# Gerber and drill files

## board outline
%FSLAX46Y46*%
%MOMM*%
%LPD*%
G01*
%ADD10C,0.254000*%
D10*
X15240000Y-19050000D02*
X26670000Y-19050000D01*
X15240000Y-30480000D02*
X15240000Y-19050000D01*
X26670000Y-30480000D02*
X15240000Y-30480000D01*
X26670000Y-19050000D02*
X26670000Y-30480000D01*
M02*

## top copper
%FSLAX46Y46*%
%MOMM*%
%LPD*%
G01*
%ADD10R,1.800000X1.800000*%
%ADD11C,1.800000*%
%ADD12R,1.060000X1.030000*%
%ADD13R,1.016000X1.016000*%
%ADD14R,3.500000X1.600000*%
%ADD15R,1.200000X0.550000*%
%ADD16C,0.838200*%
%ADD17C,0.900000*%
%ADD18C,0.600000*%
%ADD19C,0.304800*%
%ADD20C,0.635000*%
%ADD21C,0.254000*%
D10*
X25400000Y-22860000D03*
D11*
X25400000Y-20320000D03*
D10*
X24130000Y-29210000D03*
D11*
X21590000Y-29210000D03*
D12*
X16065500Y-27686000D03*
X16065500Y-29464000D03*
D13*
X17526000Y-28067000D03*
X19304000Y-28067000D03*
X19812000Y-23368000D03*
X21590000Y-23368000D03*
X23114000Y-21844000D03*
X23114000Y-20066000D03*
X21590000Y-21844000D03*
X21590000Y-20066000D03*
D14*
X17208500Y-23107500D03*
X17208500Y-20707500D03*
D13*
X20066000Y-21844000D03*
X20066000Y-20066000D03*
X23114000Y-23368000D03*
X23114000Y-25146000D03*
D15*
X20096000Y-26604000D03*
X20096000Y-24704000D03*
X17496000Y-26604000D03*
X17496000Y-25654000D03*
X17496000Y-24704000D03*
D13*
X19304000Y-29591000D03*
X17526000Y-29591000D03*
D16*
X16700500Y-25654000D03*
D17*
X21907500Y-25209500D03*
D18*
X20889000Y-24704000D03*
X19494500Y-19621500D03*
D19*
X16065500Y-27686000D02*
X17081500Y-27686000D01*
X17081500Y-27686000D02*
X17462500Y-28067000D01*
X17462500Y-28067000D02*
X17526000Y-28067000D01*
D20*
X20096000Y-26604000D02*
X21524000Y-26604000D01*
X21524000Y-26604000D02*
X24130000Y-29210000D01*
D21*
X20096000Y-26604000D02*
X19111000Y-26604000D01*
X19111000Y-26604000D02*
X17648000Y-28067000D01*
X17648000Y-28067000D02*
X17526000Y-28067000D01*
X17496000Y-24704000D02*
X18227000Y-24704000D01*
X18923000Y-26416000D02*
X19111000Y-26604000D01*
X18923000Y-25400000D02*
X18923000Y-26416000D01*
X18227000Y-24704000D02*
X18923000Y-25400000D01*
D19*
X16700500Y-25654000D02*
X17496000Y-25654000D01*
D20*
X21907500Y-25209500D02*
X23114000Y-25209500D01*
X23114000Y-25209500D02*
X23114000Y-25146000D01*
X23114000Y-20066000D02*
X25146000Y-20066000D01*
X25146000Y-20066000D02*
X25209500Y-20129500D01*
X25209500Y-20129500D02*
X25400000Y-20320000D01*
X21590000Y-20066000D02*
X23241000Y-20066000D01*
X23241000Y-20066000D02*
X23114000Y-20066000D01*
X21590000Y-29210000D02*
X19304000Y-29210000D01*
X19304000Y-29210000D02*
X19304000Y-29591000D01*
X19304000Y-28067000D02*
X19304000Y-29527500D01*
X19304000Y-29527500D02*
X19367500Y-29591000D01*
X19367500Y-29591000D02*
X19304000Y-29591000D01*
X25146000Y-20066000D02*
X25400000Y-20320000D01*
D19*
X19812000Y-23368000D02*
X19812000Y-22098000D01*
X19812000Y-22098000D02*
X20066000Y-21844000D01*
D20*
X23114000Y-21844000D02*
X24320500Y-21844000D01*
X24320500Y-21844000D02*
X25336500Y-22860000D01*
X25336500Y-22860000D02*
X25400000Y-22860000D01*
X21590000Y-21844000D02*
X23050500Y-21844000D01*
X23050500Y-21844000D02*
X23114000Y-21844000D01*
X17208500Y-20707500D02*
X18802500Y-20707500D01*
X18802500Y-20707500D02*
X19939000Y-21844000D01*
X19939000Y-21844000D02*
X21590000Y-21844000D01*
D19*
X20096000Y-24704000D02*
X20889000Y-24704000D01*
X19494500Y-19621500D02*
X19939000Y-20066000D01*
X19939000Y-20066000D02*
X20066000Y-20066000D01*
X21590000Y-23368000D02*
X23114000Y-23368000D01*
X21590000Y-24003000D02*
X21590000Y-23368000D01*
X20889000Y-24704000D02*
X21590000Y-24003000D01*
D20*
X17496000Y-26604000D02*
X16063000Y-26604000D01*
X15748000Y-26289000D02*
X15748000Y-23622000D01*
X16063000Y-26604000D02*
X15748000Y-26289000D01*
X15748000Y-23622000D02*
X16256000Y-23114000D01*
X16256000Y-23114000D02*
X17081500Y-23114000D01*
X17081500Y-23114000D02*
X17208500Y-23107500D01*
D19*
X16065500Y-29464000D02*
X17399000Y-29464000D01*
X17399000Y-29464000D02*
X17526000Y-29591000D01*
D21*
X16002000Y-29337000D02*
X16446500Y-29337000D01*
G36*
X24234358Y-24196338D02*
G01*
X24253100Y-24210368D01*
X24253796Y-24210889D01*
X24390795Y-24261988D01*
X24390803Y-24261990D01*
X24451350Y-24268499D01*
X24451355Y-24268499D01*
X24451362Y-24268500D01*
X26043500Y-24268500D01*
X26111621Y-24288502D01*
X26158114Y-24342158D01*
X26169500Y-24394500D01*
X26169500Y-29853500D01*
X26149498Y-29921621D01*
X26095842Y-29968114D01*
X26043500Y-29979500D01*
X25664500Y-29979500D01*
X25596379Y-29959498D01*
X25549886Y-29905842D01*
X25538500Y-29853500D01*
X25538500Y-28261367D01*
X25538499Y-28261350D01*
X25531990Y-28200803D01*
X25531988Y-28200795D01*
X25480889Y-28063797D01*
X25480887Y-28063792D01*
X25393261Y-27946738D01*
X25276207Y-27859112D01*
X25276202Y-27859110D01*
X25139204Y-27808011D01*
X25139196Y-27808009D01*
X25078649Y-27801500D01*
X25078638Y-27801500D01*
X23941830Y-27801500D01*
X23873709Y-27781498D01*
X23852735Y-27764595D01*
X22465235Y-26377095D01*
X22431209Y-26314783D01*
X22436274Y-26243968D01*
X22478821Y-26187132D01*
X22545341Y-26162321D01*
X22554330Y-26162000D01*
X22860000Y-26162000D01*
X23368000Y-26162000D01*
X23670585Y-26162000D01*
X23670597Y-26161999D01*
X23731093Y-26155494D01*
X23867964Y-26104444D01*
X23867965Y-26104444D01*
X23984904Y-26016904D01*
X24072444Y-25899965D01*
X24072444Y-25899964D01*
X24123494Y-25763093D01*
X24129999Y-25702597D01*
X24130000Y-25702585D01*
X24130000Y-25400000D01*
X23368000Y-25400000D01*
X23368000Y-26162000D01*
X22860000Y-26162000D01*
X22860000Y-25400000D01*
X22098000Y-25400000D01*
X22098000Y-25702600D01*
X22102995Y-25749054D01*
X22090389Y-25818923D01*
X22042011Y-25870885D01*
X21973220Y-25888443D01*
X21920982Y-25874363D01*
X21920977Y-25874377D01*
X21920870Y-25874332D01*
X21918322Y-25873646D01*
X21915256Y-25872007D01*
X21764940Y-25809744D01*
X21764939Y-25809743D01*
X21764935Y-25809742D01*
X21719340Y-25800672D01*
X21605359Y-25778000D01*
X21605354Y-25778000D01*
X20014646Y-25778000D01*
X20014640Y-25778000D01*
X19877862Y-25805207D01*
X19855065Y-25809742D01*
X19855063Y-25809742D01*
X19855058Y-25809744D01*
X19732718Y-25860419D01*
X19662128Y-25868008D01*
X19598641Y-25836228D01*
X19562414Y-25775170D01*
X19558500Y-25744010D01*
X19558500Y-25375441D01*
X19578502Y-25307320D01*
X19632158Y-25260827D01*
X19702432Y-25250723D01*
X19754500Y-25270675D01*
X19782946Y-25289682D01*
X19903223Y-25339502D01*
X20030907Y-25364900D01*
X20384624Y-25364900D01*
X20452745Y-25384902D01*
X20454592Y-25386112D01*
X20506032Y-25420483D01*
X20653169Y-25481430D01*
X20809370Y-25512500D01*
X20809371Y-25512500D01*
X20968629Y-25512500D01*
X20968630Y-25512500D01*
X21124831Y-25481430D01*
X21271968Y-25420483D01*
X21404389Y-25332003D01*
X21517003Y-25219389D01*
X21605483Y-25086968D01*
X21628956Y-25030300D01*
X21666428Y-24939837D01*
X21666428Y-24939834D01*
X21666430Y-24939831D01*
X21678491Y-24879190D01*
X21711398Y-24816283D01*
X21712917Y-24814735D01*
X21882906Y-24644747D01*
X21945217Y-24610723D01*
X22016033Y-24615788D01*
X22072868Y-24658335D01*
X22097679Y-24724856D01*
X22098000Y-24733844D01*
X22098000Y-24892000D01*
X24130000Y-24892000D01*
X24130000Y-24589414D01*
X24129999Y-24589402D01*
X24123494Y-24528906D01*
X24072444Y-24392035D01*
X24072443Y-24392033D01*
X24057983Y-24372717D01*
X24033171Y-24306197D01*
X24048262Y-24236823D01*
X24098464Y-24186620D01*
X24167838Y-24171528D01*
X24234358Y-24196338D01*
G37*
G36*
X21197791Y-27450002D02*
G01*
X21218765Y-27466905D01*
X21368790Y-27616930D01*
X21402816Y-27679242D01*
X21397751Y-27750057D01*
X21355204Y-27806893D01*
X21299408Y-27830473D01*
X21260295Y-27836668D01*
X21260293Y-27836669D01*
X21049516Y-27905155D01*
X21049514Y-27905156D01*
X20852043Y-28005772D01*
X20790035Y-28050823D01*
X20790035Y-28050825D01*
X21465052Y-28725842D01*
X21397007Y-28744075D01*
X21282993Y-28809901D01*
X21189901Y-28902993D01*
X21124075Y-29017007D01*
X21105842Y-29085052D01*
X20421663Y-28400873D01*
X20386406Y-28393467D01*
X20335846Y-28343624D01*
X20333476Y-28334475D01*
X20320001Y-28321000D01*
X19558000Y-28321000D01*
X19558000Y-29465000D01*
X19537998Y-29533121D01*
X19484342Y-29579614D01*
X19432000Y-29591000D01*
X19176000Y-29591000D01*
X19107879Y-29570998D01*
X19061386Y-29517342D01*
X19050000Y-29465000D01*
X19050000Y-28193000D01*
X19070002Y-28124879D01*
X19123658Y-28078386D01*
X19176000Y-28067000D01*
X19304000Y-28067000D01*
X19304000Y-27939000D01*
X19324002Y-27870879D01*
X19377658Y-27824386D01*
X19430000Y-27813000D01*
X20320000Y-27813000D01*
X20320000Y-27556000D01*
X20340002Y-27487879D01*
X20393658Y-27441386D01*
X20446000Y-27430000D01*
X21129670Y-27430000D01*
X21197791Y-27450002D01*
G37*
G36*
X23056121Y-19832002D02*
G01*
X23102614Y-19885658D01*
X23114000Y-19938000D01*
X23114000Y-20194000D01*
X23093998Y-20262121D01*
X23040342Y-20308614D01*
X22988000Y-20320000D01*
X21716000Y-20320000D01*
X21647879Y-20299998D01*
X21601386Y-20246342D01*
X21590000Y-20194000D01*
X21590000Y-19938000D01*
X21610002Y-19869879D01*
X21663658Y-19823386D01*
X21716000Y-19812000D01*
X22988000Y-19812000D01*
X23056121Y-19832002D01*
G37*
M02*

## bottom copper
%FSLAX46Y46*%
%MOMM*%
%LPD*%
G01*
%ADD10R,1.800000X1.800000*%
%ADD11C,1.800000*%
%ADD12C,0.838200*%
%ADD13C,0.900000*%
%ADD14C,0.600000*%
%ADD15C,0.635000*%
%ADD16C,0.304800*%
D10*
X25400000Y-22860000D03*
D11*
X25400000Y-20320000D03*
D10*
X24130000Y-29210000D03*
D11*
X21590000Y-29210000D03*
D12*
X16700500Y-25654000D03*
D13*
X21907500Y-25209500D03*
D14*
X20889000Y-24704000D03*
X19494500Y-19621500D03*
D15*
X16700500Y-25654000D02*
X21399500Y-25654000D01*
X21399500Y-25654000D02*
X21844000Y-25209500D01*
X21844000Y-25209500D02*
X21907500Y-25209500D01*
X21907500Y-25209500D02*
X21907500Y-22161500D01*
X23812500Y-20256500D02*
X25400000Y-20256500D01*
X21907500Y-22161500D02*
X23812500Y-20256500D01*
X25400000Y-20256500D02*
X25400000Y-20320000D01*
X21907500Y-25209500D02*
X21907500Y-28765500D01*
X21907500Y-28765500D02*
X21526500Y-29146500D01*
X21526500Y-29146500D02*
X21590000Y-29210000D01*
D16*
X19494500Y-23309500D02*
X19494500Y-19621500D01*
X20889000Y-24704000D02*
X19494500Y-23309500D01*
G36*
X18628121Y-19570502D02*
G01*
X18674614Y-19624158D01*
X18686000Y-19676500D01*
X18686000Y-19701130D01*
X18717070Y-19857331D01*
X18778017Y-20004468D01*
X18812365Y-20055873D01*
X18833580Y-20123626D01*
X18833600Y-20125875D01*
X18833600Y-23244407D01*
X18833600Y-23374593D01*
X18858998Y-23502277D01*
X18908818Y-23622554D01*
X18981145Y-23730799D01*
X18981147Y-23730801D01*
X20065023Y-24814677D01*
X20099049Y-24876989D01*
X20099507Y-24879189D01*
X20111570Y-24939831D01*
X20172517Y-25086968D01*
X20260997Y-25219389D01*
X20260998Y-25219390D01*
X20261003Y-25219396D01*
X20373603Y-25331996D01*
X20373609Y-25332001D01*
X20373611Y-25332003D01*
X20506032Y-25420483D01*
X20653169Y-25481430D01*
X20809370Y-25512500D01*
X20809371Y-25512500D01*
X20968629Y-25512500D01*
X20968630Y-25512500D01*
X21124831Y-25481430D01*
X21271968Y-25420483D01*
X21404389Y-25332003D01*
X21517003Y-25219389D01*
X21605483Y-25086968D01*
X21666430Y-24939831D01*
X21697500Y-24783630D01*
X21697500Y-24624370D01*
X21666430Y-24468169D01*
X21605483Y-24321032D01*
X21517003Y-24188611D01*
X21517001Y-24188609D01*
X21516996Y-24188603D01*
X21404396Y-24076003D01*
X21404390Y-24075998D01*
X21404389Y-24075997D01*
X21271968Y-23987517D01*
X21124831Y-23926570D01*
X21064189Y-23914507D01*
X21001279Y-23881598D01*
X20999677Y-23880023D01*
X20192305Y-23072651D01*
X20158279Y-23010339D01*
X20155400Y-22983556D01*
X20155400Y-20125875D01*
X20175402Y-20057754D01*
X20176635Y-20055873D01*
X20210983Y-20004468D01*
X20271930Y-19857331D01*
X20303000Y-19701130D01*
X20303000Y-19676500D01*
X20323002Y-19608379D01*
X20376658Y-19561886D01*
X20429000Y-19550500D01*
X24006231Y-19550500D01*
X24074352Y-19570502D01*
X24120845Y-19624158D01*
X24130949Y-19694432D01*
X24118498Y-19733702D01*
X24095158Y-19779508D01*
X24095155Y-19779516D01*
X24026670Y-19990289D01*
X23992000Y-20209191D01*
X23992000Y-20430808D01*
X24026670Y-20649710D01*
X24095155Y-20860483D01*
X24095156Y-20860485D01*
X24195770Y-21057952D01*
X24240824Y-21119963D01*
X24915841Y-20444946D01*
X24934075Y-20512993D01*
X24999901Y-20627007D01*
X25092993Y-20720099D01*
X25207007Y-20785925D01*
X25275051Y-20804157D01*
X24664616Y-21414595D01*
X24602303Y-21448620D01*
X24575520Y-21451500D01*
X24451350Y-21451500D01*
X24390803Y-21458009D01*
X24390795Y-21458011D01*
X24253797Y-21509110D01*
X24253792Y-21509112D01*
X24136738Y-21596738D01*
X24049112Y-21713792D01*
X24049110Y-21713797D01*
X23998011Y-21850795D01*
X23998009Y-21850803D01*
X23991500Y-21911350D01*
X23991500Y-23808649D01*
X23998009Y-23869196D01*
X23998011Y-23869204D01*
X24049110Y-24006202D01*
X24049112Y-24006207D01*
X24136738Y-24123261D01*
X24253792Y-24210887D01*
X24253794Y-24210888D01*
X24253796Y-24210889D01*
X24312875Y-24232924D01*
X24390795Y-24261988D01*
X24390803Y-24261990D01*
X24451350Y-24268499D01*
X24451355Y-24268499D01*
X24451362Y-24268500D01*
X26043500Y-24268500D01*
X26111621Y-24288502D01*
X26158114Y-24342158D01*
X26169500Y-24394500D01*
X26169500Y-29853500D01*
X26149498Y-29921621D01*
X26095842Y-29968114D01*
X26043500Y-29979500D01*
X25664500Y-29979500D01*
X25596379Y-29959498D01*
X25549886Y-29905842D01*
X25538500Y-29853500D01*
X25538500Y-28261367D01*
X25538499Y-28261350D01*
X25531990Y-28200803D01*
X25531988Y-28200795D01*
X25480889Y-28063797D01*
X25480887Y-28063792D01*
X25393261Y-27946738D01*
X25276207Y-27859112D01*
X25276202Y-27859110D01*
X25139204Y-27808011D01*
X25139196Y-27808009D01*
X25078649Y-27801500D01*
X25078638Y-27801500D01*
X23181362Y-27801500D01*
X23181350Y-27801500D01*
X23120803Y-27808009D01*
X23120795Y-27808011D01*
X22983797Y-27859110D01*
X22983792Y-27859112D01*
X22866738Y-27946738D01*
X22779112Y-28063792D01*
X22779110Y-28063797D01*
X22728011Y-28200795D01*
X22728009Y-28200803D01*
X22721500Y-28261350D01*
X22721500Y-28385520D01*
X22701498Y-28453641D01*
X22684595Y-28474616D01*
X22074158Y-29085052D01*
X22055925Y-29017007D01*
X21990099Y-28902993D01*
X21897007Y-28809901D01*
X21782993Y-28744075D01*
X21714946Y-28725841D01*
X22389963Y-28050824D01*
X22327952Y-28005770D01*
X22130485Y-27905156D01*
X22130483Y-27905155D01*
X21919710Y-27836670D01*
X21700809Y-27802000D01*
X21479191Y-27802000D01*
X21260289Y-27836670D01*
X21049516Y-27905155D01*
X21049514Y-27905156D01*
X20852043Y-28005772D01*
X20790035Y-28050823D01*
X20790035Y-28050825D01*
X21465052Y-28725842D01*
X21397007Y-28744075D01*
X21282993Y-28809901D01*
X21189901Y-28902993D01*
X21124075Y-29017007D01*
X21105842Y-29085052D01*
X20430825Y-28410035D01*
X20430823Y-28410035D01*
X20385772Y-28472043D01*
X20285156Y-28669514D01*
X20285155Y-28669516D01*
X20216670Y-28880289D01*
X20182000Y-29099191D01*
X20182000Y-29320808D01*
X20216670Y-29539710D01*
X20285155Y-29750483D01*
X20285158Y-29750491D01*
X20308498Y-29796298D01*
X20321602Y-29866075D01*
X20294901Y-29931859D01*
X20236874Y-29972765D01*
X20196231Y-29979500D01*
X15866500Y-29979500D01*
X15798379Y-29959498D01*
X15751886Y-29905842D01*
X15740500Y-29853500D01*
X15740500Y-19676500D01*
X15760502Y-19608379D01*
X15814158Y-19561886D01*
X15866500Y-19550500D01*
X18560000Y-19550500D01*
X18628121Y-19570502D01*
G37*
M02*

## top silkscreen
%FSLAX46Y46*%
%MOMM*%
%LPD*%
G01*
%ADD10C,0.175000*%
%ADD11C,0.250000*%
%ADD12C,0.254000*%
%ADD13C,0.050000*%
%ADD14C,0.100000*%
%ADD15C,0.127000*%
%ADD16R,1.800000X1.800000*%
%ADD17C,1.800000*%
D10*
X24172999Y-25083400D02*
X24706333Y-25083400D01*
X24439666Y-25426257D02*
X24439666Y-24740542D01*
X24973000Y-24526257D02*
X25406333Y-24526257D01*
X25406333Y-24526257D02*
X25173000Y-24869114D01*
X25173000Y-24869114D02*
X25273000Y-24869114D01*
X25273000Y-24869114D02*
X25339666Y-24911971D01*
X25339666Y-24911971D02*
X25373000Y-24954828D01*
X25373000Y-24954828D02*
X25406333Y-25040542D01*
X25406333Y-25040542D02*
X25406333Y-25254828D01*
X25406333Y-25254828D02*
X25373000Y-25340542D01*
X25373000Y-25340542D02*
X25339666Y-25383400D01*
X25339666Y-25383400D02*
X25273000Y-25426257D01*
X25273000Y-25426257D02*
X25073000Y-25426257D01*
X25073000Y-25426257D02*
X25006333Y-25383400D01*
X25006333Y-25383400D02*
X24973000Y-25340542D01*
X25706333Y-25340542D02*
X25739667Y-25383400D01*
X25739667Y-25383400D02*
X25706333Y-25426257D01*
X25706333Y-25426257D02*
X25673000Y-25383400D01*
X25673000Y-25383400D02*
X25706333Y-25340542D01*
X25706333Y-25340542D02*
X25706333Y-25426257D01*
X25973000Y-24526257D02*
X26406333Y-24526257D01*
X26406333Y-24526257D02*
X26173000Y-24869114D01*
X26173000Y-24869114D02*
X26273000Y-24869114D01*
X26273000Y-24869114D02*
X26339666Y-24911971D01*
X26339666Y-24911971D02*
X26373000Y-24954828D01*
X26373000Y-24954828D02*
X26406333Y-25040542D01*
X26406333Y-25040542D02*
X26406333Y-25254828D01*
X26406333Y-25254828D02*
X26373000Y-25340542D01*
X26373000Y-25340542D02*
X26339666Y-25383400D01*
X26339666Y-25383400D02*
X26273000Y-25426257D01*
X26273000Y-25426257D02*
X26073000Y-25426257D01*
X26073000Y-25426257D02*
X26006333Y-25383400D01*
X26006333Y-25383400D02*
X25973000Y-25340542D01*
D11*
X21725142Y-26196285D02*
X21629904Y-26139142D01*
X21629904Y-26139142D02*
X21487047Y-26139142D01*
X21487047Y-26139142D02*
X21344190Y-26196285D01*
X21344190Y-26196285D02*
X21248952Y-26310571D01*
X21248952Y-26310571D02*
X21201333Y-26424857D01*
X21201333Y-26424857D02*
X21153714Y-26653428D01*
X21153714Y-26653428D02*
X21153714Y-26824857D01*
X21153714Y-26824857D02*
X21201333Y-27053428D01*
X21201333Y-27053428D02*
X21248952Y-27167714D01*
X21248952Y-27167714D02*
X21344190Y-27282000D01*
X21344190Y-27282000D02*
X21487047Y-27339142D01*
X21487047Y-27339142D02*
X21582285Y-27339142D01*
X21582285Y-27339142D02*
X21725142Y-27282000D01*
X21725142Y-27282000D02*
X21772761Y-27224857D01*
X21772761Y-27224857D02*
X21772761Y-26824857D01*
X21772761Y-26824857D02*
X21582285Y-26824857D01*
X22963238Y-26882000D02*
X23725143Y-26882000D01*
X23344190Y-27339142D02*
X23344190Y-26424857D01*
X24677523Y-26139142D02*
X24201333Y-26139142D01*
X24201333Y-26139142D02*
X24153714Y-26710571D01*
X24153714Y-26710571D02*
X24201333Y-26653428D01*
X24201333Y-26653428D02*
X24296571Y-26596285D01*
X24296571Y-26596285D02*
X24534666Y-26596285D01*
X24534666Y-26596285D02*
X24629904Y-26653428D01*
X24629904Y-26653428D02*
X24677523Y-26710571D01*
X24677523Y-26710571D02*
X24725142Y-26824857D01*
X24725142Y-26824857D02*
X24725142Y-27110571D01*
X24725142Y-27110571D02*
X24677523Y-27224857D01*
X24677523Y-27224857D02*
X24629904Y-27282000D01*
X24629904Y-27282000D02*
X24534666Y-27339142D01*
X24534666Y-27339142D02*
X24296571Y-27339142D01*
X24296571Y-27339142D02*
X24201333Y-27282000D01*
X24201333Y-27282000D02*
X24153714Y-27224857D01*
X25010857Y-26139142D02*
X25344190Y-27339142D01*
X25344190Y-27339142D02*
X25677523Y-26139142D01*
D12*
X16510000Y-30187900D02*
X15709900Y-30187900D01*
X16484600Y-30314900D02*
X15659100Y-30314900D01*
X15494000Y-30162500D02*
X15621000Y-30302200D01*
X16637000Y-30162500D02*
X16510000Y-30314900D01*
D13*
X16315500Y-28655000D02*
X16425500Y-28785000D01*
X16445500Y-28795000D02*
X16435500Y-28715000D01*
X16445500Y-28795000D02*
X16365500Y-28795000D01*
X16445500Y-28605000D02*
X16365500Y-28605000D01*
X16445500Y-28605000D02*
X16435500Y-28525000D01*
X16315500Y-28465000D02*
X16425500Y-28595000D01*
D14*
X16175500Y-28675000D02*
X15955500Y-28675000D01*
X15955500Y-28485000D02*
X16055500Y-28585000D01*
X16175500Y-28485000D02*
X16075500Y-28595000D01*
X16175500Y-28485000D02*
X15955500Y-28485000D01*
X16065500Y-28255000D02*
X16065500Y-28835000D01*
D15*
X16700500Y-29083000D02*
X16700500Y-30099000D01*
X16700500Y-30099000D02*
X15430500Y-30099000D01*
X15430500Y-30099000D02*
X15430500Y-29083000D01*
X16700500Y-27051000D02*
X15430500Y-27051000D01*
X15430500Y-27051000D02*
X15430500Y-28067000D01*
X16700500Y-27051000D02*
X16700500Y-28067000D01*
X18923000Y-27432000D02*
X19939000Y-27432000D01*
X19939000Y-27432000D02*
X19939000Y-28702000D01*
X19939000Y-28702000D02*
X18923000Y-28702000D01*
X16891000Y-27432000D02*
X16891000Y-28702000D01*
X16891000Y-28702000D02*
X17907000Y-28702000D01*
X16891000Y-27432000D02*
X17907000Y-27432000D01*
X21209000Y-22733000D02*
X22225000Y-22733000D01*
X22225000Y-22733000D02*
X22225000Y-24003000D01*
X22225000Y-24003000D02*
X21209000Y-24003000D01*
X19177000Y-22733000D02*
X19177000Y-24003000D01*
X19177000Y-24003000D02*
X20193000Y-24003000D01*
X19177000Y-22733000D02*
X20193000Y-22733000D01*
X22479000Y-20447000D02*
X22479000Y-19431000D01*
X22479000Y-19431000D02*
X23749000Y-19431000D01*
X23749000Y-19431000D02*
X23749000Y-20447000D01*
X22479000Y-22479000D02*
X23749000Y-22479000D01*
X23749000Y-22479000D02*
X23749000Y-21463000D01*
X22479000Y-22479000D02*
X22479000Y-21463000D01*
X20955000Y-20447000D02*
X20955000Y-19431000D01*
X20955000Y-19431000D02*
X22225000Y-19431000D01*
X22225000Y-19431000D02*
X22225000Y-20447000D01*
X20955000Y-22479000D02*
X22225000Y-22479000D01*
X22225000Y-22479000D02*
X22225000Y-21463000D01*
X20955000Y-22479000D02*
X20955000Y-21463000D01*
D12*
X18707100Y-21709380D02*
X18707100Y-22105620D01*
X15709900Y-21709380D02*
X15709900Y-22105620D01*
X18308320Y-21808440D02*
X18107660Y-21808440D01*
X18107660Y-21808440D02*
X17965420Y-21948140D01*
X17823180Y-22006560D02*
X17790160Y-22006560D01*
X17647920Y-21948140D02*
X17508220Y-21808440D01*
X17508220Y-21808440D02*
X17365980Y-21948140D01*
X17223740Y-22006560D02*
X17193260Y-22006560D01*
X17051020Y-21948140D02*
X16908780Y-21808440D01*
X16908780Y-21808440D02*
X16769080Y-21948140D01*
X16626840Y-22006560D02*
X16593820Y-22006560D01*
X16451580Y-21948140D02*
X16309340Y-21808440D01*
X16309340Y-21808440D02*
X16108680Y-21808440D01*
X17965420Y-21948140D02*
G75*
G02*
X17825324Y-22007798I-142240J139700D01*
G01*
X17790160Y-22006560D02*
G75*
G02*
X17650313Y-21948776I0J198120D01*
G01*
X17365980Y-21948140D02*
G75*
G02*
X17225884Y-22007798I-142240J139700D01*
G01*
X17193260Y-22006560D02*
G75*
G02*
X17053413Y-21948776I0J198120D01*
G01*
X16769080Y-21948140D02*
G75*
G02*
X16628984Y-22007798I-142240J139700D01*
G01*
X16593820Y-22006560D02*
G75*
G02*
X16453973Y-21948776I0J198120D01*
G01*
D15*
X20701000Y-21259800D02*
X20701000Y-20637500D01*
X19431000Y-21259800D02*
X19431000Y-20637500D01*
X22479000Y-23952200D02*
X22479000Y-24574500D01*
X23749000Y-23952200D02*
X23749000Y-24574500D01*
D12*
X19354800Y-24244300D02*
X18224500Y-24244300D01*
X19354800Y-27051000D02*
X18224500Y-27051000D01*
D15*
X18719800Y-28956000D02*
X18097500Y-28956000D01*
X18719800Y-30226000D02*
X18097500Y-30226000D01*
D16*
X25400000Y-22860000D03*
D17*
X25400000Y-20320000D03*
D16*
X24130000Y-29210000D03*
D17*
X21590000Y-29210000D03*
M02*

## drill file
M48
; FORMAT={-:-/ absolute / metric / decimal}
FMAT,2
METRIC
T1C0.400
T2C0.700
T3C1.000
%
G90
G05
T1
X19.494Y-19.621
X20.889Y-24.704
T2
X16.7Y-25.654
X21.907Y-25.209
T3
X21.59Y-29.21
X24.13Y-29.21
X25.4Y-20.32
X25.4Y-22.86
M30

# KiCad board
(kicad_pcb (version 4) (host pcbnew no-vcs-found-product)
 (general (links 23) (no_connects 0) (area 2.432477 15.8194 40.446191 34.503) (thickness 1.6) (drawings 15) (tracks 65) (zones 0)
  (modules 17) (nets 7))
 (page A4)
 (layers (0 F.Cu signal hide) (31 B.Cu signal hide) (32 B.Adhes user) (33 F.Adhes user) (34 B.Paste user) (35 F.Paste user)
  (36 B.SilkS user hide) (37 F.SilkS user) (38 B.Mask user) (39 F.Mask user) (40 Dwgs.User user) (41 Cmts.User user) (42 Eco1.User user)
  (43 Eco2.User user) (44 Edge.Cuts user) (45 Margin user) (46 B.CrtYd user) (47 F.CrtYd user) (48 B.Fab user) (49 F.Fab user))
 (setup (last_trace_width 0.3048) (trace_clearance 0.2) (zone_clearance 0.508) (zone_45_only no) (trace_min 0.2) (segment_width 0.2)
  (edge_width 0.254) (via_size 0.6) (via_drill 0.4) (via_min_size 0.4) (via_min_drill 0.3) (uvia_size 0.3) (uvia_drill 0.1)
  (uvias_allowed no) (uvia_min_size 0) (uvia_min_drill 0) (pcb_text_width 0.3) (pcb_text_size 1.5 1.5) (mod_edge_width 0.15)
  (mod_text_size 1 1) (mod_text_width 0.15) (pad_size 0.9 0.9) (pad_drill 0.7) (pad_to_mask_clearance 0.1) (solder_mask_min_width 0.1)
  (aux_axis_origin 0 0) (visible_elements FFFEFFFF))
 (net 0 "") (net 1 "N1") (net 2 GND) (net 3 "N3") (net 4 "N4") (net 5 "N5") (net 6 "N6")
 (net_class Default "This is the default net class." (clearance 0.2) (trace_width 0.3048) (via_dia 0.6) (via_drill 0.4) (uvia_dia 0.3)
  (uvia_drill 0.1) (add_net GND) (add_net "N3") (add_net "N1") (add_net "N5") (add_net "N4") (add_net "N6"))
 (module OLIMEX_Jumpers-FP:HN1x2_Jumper (layer F.Cu) (at 25.4 21.59 90)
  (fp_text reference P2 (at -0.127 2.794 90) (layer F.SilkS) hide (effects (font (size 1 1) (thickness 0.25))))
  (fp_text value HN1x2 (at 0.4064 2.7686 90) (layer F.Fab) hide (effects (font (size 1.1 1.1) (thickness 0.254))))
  (pad 1 thru_hole rect (at -1.27 0 180) (size 1.8 1.8) (drill 1) (layers *.Cu *.Mask F.SilkS) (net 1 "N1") (solder_mask_margin 0.0508)
   (solder_paste_margin -0.0508))
  (pad 2 thru_hole circle (at 1.27 0 180) (size 1.8 1.8) (drill 1) (layers *.Cu *.Mask F.SilkS) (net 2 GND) (solder_mask_margin 0.0508)
   (solder_paste_margin -0.0508)))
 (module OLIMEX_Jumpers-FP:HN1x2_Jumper (layer F.Cu) (at 22.86 29.21 180)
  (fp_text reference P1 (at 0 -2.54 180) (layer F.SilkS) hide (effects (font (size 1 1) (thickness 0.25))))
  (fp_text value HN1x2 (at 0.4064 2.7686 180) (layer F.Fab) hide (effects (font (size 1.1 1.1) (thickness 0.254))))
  (pad 1 thru_hole rect (at -1.27 0 270) (size 1.8 1.8) (drill 1) (layers *.Cu *.Mask F.SilkS) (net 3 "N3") (solder_mask_margin 0.0508)
   (solder_paste_margin -0.0508))
  (pad 2 thru_hole circle (at 1.27 0 270) (size 1.8 1.8) (drill 1) (layers *.Cu *.Mask F.SilkS) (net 2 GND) (solder_mask_margin 0.0508)
   (solder_paste_margin -0.0508)))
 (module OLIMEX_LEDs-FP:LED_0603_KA (layer F.Cu) (at 16.0655 28.575 270)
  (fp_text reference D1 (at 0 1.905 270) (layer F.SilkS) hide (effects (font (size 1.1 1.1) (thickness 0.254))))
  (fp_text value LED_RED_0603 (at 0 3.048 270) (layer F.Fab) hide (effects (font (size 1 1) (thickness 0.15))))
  (fp_line (start 1.6129 -0.4445) (end 1.6129 0.3556) (layer F.SilkS) (width 0.254))
  (fp_line (start 1.7399 -0.4191) (end 1.7399 0.4064) (layer F.SilkS) (width 0.254))
  (fp_line (start 1.5875 0.5715) (end 1.7272 0.4445) (layer F.SilkS) (width 0.254))
  (fp_line (start 1.5875 -0.5715) (end 1.7399 -0.4445) (layer F.SilkS) (width 0.254))
  (fp_line (start 0.08 -0.25) (end 0.21 -0.36) (layer F.SilkS) (width 0.05))
  (fp_line (start 0.22 -0.38) (end 0.14 -0.37) (layer F.SilkS) (width 0.05))
  (fp_line (start 0.22 -0.38) (end 0.22 -0.3) (layer F.SilkS) (width 0.05))
  (fp_line (start 0.03 -0.38) (end 0.03 -0.3) (layer F.SilkS) (width 0.05))
  (fp_line (start 0.03 -0.38) (end -0.05 -0.37) (layer F.SilkS) (width 0.05))
  (fp_line (start -0.11 -0.25) (end 0.02 -0.36) (layer F.SilkS) (width 0.05))
  (fp_line (start 0.1 -0.11) (end 0.1 0.11) (layer F.SilkS) (width 0.1))
  (fp_line (start -0.09 0.11) (end 0.01 0.01) (layer F.SilkS) (width 0.1))
  (fp_line (start -0.09 -0.11) (end 0.02 -0.01) (layer F.SilkS) (width 0.1))
  (fp_line (start -0.09 -0.11) (end -0.09 0.11) (layer F.SilkS) (width 0.1))
  (fp_line (start -0.32 0) (end 0.26 0) (layer F.SilkS) (width 0.1))
  (fp_line (start 0.508 -0.635) (end 1.524 -0.635) (layer F.SilkS) (width 0.127))
  (fp_line (start 1.524 -0.635) (end 1.524 0.635) (layer F.SilkS) (width 0.127))
  (fp_line (start 1.524 0.635) (end 0.508 0.635) (layer F.SilkS) (width 0.127))
  (fp_line (start -1.524 -0.635) (end -1.524 0.635) (layer F.SilkS) (width 0.127))
  (fp_line (start -1.524 0.635) (end -0.508 0.635) (layer F.SilkS) (width 0.127))
  (fp_line (start -1.524 -0.635) (end -0.508 -0.635) (layer F.SilkS) (width 0.127))
  (pad 2 smd rect (at -0.889 0 270) (size 1.03 1.06) (layers F.Cu F.Paste F.Mask) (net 3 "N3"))
  (pad 1 smd rect (at 0.889 0 270) (size 1.03 1.06) (layers F.Cu F.Paste F.Mask) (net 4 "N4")))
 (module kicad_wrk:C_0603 (layer F.Cu) (at 18.415 28.067)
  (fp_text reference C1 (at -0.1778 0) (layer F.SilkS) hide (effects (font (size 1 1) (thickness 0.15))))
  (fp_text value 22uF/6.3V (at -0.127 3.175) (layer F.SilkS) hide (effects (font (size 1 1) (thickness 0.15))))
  (fp_line (start 0.508 -0.635) (end 1.524 -0.635) (layer F.SilkS) (width 0.127))
  (fp_line (start 1.524 -0.635) (end 1.524 0.635) (layer F.SilkS) (width 0.127))
  (fp_line (start 1.524 0.635) (end 0.508 0.635) (layer F.SilkS) (width 0.127))
  (fp_line (start -1.524 -0.635) (end -1.524 0.635) (layer F.SilkS) (width 0.127))
  (fp_line (start -1.524 0.635) (end -0.508 0.635) (layer F.SilkS) (width 0.127))
  (fp_line (start -1.524 -0.635) (end -0.508 -0.635) (layer F.SilkS) (width 0.127))
  (pad 1 smd rect (at -0.889 0) (size 1.016 1.016) (layers F.Cu F.Paste F.Mask) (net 3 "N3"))
  (pad 2 smd rect (at 0.889 0) (size 1.016 1.016) (layers F.Cu F.Paste F.Mask) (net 2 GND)))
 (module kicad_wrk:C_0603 (layer F.Cu) (at 20.701 23.368)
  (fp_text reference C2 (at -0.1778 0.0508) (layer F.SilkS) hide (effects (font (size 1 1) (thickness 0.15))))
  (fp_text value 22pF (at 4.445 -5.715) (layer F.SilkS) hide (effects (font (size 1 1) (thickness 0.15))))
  (fp_line (start 0.508 -0.635) (end 1.524 -0.635) (layer F.SilkS) (width 0.127))
  (fp_line (start 1.524 -0.635) (end 1.524 0.635) (layer F.SilkS) (width 0.127))
  (fp_line (start 1.524 0.635) (end 0.508 0.635) (layer F.SilkS) (width 0.127))
  (fp_line (start -1.524 -0.635) (end -1.524 0.635) (layer F.SilkS) (width 0.127))
  (fp_line (start -1.524 0.635) (end -0.508 0.635) (layer F.SilkS) (width 0.127))
  (fp_line (start -1.524 -0.635) (end -0.508 -0.635) (layer F.SilkS) (width 0.127))
  (pad 1 smd rect (at -0.889 0) (size 1.016 1.016) (layers F.Cu F.Paste F.Mask) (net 1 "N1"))
  (pad 2 smd rect (at 0.889 0) (size 1.016 1.016) (layers F.Cu F.Paste F.Mask) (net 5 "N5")))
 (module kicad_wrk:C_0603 (layer F.Cu) (at 23.114 20.955 90)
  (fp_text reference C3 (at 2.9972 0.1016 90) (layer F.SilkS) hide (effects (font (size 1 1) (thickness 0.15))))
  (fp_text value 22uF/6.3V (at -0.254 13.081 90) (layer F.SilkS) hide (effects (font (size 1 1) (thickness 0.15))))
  (fp_line (start 0.508 -0.635) (end 1.524 -0.635) (layer F.SilkS) (width 0.127))
  (fp_line (start 1.524 -0.635) (end 1.524 0.635) (layer F.SilkS) (width 0.127))
  (fp_line (start 1.524 0.635) (end 0.508 0.635) (layer F.SilkS) (width 0.127))
  (fp_line (start -1.524 -0.635) (end -1.524 0.635) (layer F.SilkS) (width 0.127))
  (fp_line (start -1.524 0.635) (end -0.508 0.635) (layer F.SilkS) (width 0.127))
  (fp_line (start -1.524 -0.635) (end -0.508 -0.635) (layer F.SilkS) (width 0.127))
  (pad 1 smd rect (at -0.889 0 90) (size 1.016 1.016) (layers F.Cu F.Paste F.Mask) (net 1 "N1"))
  (pad 2 smd rect (at 0.889 0 90) (size 1.016 1.016) (layers F.Cu F.Paste F.Mask) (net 2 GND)))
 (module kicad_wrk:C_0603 (layer F.Cu) (at 21.59 20.955 90)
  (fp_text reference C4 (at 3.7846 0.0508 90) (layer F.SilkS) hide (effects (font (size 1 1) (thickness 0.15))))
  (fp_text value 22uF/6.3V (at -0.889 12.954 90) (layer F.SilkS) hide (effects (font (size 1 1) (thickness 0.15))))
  (fp_line (start 0.508 -0.635) (end 1.524 -0.635) (layer F.SilkS) (width 0.127))
  (fp_line (start 1.524 -0.635) (end 1.524 0.635) (layer F.SilkS) (width 0.127))
  (fp_line (start 1.524 0.635) (end 0.508 0.635) (layer F.SilkS) (width 0.127))
  (fp_line (start -1.524 -0.635) (end -1.524 0.635) (layer F.SilkS) (width 0.127))
  (fp_line (start -1.524 0.635) (end -0.508 0.635) (layer F.SilkS) (width 0.127))
  (fp_line (start -1.524 -0.635) (end -0.508 -0.635) (layer F.SilkS) (width 0.127))
  (pad 1 smd rect (at -0.889 0 90) (size 1.016 1.016) (layers F.Cu F.Paste F.Mask) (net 1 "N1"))
  (pad 2 smd rect (at 0.889 0 90) (size 1.016 1.016) (layers F.Cu F.Paste F.Mask) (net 2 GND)))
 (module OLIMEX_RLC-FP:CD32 (layer F.Cu) (at 17.2085 21.9075 90)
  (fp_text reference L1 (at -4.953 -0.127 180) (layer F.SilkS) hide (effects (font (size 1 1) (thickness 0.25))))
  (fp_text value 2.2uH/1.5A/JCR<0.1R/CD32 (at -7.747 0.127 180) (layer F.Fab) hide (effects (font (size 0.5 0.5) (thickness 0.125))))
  (fp_line (start 0.19812 1.4986) (end -0.19812 1.4986) (layer F.SilkS) (width 0.254))
  (fp_line (start 0.19812 -1.4986) (end -0.19812 -1.4986) (layer F.SilkS) (width 0.254))
  (fp_line (start 0.09906 1.09982) (end 0.09906 0.89916) (layer F.SilkS) (width 0.254))
  (fp_line (start 0.09906 0.89916) (end -0.04064 0.75692) (layer F.SilkS) (width 0.254))
  (fp_line (start -0.09906 0.61468) (end -0.09906 0.58166) (layer F.SilkS) (width 0.254))
  (fp_line (start -0.04064 0.43942) (end 0.09906 0.29972) (layer F.SilkS) (width 0.254))
  (fp_line (start 0.09906 0.29972) (end -0.04064 0.15748) (layer F.SilkS) (width 0.254))
  (fp_line (start -0.09906 0.01524) (end -0.09906 -0.01524) (layer F.SilkS) (width 0.254))
  (fp_line (start -0.04064 -0.15748) (end 0.09906 -0.29972) (layer F.SilkS) (width 0.254))
  (fp_line (start 0.09906 -0.29972) (end -0.04064 -0.43942) (layer F.SilkS) (width 0.254))
  (fp_line (start -0.09906 -0.58166) (end -0.09906 -0.61468) (layer F.SilkS) (width 0.254))
  (fp_line (start -0.04064 -0.75692) (end 0.09906 -0.89916) (layer F.SilkS) (width 0.254))
  (fp_line (start 0.09906 -0.89916) (end 0.09906 -1.09982) (layer F.SilkS) (width 0.254))
  (fp_arc (start 0.09906 0.61468) (end -0.04064 0.75692) (angle 44.9) (layer F.SilkS) (width 0.254))
  (fp_arc (start 0.09906 0.58166) (end -0.09906 0.58166) (angle 44.9) (layer F.SilkS) (width 0.254))
  (fp_arc (start 0.09906 0.01524) (end -0.04064 0.15748) (angle 44.9) (layer F.SilkS) (width 0.254))
  (fp_arc (start 0.09906 -0.01524) (end -0.09906 -0.01524) (angle 44.9) (layer F.SilkS) (width 0.254))
  (fp_arc (start 0.09906 -0.58166) (end -0.04064 -0.43942) (angle 44.9) (layer F.SilkS) (width 0.254))
  (fp_arc (start 0.09906 -0.61468) (end -0.09906 -0.61468) (angle 44.9) (layer F.SilkS) (width 0.254))
  (pad 1 smd rect (at -1.2 0 180) (size 3.5 1.6) (layers F.Cu F.Paste F.Mask) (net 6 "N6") (solder_mask_margin 0.0508)
   (solder_paste_margin -0.0508) (clearance 0.0508))
  (pad 2 smd rect (at 1.2 0 180) (size 3.5 1.6) (layers F.Cu F.Paste F.Mask) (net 1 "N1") (solder_mask_margin 0.0508)
   (solder_paste_margin -0.0508) (clearance 0.0508)))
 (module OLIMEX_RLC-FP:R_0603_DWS (layer F.Cu) (at 20.066 20.955 90)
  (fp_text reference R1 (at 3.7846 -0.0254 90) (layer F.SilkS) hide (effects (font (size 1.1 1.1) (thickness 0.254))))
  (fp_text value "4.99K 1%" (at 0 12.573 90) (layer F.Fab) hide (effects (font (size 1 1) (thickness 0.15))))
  (fp_line (start -0.3048 0.635) (end 0.3175 0.635) (layer F.SilkS) (width 0.127))
  (fp_line (start -0.3048 -0.635) (end 0.3175 -0.635) (layer F.SilkS) (width 0.127))
  (pad 1 smd rect (at -0.889 0 90) (size 1.016 1.016) (layers F.Cu F.Paste F.Mask) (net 1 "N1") (solder_mask_margin 0.0508)
   (solder_paste_margin -0.0508) (clearance 0.0508))
  (pad 2 smd rect (at 0.889 0 90) (size 1.016 1.016) (layers F.Cu F.Paste F.Mask) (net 5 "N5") (solder_mask_margin 0.0508)
   (solder_paste_margin -0.0508) (clearance 0.0508)))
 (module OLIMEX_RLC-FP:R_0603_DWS (layer F.Cu) (at 23.114 24.257 270)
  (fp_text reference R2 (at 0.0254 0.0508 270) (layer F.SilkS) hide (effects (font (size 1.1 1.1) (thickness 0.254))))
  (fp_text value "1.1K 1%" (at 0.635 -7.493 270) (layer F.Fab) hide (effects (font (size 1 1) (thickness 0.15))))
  (fp_line (start -0.3048 0.635) (end 0.3175 0.635) (layer F.SilkS) (width 0.127))
  (fp_line (start -0.3048 -0.635) (end 0.3175 -0.635) (layer F.SilkS) (width 0.127))
  (pad 1 smd rect (at -0.889 0 270) (size 1.016 1.016) (layers F.Cu F.Paste F.Mask) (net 5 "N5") (solder_mask_margin 0.0508)
   (solder_paste_margin -0.0508) (clearance 0.0508))
  (pad 2 smd rect (at 0.889 0 270) (size 1.016 1.016) (layers F.Cu F.Paste F.Mask) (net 2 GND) (solder_mask_margin 0.0508)
   (solder_paste_margin -0.0508) (clearance 0.0508)))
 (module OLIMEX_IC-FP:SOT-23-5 (layer F.Cu) (at 18.796 25.654 180)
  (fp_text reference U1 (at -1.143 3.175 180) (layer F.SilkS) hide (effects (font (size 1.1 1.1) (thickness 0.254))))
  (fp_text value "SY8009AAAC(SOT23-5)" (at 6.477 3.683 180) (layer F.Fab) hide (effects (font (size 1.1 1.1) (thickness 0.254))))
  (fp_line (start -0.5588 1.4097) (end 0.5715 1.4097) (layer F.SilkS) (width 0.254))
  (fp_line (start -0.5588 -1.397) (end 0.5715 -1.397) (layer F.SilkS) (width 0.254))
  (pad 4 smd rect (at -1.3 -0.95 180) (size 1.2 0.55) (layers F.Cu F.Paste F.Mask) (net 3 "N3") (solder_mask_margin 0.0508)
   (solder_paste_margin -0.0508) (clearance 0.0508))
  (pad 5 smd rect (at -1.3 0.95 180) (size 1.2 0.55) (layers F.Cu F.Paste F.Mask) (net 5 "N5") (solder_mask_margin 0.0508)
   (solder_paste_margin -0.0508) (clearance 0.0508))
  (pad 3 smd rect (at 1.3 -0.95 180) (size 1.2 0.55) (layers F.Cu F.Paste F.Mask) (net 6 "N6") (solder_mask_margin 0.0508)
   (solder_paste_margin -0.0508) (clearance 0.0508))
  (pad 2 smd rect (at 1.3 0 180) (size 1.2 0.55) (layers F.Cu F.Paste F.Mask) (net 2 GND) (solder_mask_margin 0.0508)
   (solder_paste_margin -0.0508) (clearance 0.0508))
  (pad 1 smd rect (at 1.3 0.95 180) (size 1.2 0.55) (layers F.Cu F.Paste F.Mask) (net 3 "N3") (solder_mask_margin 0.0508)
   (solder_paste_margin -0.0508) (clearance 0.0508)))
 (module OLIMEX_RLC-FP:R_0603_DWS (layer F.Cu) (at 18.415 29.591 180)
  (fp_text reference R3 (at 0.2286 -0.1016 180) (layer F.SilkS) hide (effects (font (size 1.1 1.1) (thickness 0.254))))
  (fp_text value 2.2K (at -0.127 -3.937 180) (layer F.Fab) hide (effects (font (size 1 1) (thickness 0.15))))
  (fp_line (start -0.3048 0.635) (end 0.3175 0.635) (layer F.SilkS) (width 0.127))
  (fp_line (start -0.3048 -0.635) (end 0.3175 -0.635) (layer F.SilkS) (width 0.127))
  (pad 1 smd rect (at -0.889 0 180) (size 1.016 1.016) (layers F.Cu F.Paste F.Mask) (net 2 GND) (solder_mask_margin 0.0508)
   (solder_paste_margin -0.0508) (clearance 0.0508))
  (pad 2 smd rect (at 0.889 0 180) (size 1.016 1.016) (layers F.Cu F.Paste F.Mask) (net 4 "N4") (solder_mask_margin 0.0508)
   (solder_paste_margin -0.0508) (clearance 0.0508)))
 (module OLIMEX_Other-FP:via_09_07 (layer F.Cu) (at 16.7005 25.654)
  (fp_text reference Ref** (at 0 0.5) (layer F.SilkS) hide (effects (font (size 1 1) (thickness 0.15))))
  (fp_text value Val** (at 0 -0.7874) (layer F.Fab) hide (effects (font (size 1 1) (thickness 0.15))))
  (pad 0 thru_hole circle (at 0 0) (size 0.8382 0.8382) (drill 0.7) (layers *.Cu) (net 2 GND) (zone_connect 2)))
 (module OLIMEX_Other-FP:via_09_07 (layer F.Cu) (at 21.9075 25.273)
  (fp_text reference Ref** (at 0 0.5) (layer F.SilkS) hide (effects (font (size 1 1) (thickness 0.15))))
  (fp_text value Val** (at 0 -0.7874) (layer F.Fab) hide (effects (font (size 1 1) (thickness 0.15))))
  (pad 0 thru_hole circle (at 0 -0.0635) (size 0.9 0.9) (drill 0.7) (layers *.Cu) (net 2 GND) (zone_connect 2)))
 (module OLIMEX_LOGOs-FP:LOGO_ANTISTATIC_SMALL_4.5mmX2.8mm (layer B.Cu) (at 18.4785 28.194 180)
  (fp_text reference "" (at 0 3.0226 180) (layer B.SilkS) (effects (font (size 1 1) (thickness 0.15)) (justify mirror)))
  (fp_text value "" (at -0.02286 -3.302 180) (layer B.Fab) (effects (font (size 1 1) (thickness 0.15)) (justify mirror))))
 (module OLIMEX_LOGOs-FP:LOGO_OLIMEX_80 (layer B.Cu) (at 19.939 24.3205 180)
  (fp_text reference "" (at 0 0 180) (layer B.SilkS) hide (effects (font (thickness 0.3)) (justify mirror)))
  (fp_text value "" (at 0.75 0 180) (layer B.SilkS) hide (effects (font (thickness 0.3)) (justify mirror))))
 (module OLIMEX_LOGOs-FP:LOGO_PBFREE (layer B.Cu) (at 18.669 21.3995 180)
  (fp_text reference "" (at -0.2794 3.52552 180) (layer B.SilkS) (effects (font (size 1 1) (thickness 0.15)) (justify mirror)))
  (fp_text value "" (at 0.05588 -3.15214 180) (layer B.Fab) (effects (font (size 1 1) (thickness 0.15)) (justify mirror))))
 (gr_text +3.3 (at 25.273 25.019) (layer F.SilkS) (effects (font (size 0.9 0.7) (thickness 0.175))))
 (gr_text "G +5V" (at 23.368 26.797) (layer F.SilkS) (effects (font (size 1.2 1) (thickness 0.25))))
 (gr_line (start 15.24 19.05) (end 26.67 19.05) (angle 90) (layer Edge.Cuts) (width 0.254))
 (gr_line (start 15.24 30.48) (end 15.24 19.05) (angle 90) (layer Edge.Cuts) (width 0.254))
 (gr_line (start 26.67 30.48) (end 15.24 30.48) (angle 90) (layer Edge.Cuts) (width 0.254))
 (gr_line (start 26.67 19.05) (end 26.67 30.48) (angle 90) (layer Edge.Cuts) (width 0.254))
 (segment (start 16.0655 27.686) (end 17.0815 27.686) (width 0.3048) (layer F.Cu) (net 3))
 (segment (start 17.0815 27.686) (end 17.4625 28.067) (width 0.3048) (layer F.Cu) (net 3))
 (segment (start 17.4625 28.067) (end 17.526 28.067) (width 0.3048) (layer F.Cu) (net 3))
 (segment (start 20.096 26.604) (end 21.524 26.604) (width 0.635) (layer F.Cu) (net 3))
 (segment (start 21.524 26.604) (end 24.13 29.21) (width 0.635) (layer F.Cu) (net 3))
 (segment (start 20.096 26.604) (end 19.111 26.604) (width 0.254) (layer F.Cu) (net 3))
 (segment (start 19.111 26.604) (end 17.648 28.067) (width 0.254) (layer F.Cu) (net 3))
 (segment (start 17.648 28.067) (end 17.526 28.067) (width 0.254) (layer F.Cu) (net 3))
 (segment (start 17.496 24.704) (end 18.227 24.704) (width 0.254) (layer F.Cu) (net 3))
 (segment (start 18.923 26.416) (end 19.111 26.604) (width 0.254) (layer F.Cu) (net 3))
 (segment (start 18.923 25.4) (end 18.923 26.416) (width 0.254) (layer F.Cu) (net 3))
 (segment (start 18.227 24.704) (end 18.923 25.4) (width 0.254) (layer F.Cu) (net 3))
 (segment (start 16.7005 25.654) (end 17.496 25.654) (width 0.3048) (layer F.Cu) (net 2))
 (segment (start 16.7005 25.654) (end 21.3995 25.654) (width 0.635) (layer B.Cu) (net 2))
 (segment (start 21.3995 25.654) (end 21.844 25.2095) (width 0.635) (layer B.Cu) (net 2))
 (segment (start 21.844 25.2095) (end 21.9075 25.2095) (width 0.635) (layer B.Cu) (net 2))
 (segment (start 21.9075 25.2095) (end 21.9075 22.1615) (width 0.635) (layer B.Cu) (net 2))
 (segment (start 23.8125 20.2565) (end 25.4 20.2565) (width 0.635) (layer B.Cu) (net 2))
 (segment (start 21.9075 22.1615) (end 23.8125 20.2565) (width 0.635) (layer B.Cu) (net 2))
 (segment (start 25.4 20.2565) (end 25.4 20.32) (width 0.635) (layer B.Cu) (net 2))
 (segment (start 21.9075 25.2095) (end 21.9075 28.7655) (width 0.635) (layer B.Cu) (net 2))
 (segment (start 21.9075 28.7655) (end 21.5265 29.1465) (width 0.635) (layer B.Cu) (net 2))
 (segment (start 21.5265 29.1465) (end 21.59 29.21) (width 0.635) (layer B.Cu) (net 2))
 (segment (start 21.9075 25.2095) (end 23.114 25.2095) (width 0.635) (layer F.Cu) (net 2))
 (segment (start 23.114 25.2095) (end 23.114 25.146) (width 0.635) (layer F.Cu) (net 2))
 (segment (start 23.114 20.066) (end 25.146 20.066) (width 0.635) (layer F.Cu) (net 2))
 (segment (start 25.146 20.066) (end 25.2095 20.1295) (width 0.635) (layer F.Cu) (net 2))
 (segment (start 25.2095 20.1295) (end 25.4 20.32) (width 0.635) (layer F.Cu) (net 2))
 (segment (start 21.59 20.066) (end 23.241 20.066) (width 0.635) (layer F.Cu) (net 2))
 (segment (start 23.241 20.066) (end 23.114 20.066) (width 0.635) (layer F.Cu) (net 2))
 (segment (start 21.59 29.21) (end 19.304 29.21) (width 0.635) (layer F.Cu) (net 2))
 (segment (start 19.304 29.21) (end 19.304 29.591) (width 0.635) (layer F.Cu) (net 2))
 (segment (start 19.304 28.067) (end 19.304 29.5275) (width 0.635) (layer F.Cu) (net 2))
 (segment (start 19.304 29.5275) (end 19.3675 29.591) (width 0.635) (layer F.Cu) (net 2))
 (segment (start 19.3675 29.591) (end 19.304 29.591) (width 0.635) (layer F.Cu) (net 2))
 (segment (start 25.146 20.066) (end 25.4 20.32) (width 0.635) (layer F.Cu) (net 2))
 (segment (start 19.812 23.368) (end 19.812 22.098) (width 0.3048) (layer F.Cu) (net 1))
 (segment (start 19.812 22.098) (end 20.066 21.844) (width 0.3048) (layer F.Cu) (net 1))
 (segment (start 23.114 21.844) (end 24.3205 21.844) (width 0.635) (layer F.Cu) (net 1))
 (segment (start 24.3205 21.844) (end 25.3365 22.86) (width 0.635) (layer F.Cu) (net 1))
 (segment (start 25.3365 22.86) (end 25.4 22.86) (width 0.635) (layer F.Cu) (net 1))
 (segment (start 21.59 21.844) (end 23.0505 21.844) (width 0.635) (layer F.Cu) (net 1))
 (segment (start 23.0505 21.844) (end 23.114 21.844) (width 0.635) (layer F.Cu) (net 1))
 (segment (start 17.2085 20.7075) (end 18.8025 20.7075) (width 0.635) (layer F.Cu) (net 1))
 (segment (start 18.8025 20.7075) (end 19.939 21.844) (width 0.635) (layer F.Cu) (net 1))
 (segment (start 19.939 21.844) (end 21.59 21.844) (width 0.635) (layer F.Cu) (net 1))
 (segment (start 20.096 24.704) (end 20.889 24.704) (width 0.3048) (layer F.Cu) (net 5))
 (via (at 20.889 24.704) (size 0.6) (layers F.Cu B.Cu) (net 5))
 (segment (start 19.4945 19.6215) (end 19.939 20.066) (width 0.3048) (layer F.Cu) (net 5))
 (via (at 19.4945 19.6215) (size 0.6) (layers F.Cu B.Cu) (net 5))
 (segment (start 19.4945 23.3095) (end 19.4945 19.6215) (width 0.3048) (layer B.Cu) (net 5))
 (segment (start 20.889 24.704) (end 19.4945 23.3095) (width 0.3048) (layer B.Cu) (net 5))
 (segment (start 19.939 20.066) (end 20.066 20.066) (width 0.3048) (layer F.Cu) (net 5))
 (segment (start 21.59 23.368) (end 23.114 23.368) (width 0.3048) (layer F.Cu) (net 5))
 (segment (start 21.59 24.003) (end 21.59 23.368) (width 0.3048) (layer F.Cu) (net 5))
 (segment (start 20.889 24.704) (end 21.59 24.003) (width 0.3048) (layer F.Cu) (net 5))
 (segment (start 17.496 26.604) (end 16.063 26.604) (width 0.635) (layer F.Cu) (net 6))
 (segment (start 15.748 26.289) (end 15.748 23.622) (width 0.635) (layer F.Cu) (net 6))
 (segment (start 16.063 26.604) (end 15.748 26.289) (width 0.635) (layer F.Cu) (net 6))
 (segment (start 15.748 23.622) (end 16.256 23.114) (width 0.635) (layer F.Cu) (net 6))
 (segment (start 16.256 23.114) (end 17.0815 23.114) (width 0.635) (layer F.Cu) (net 6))
 (segment (start 17.0815 23.114) (end 17.2085 23.1075) (width 0.635) (layer F.Cu) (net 6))
 (segment (start 16.0655 29.464) (end 17.399 29.464) (width 0.3048) (layer F.Cu) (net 4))
 (segment (start 17.399 29.464) (end 17.526 29.591) (width 0.3048) (layer F.Cu) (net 4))
 (segment (start 16.002 29.337) (end 16.4465 29.337) (width 0.254) (layer F.Cu) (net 4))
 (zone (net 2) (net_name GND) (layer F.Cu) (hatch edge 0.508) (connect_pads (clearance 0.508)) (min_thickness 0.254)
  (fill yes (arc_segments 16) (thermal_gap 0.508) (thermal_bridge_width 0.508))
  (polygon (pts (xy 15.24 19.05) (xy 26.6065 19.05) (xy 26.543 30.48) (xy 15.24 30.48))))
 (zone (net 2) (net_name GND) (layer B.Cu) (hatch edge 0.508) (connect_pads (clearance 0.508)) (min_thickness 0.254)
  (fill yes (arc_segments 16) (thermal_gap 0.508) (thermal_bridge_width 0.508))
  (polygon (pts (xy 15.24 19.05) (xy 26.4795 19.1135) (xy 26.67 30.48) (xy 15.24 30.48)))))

